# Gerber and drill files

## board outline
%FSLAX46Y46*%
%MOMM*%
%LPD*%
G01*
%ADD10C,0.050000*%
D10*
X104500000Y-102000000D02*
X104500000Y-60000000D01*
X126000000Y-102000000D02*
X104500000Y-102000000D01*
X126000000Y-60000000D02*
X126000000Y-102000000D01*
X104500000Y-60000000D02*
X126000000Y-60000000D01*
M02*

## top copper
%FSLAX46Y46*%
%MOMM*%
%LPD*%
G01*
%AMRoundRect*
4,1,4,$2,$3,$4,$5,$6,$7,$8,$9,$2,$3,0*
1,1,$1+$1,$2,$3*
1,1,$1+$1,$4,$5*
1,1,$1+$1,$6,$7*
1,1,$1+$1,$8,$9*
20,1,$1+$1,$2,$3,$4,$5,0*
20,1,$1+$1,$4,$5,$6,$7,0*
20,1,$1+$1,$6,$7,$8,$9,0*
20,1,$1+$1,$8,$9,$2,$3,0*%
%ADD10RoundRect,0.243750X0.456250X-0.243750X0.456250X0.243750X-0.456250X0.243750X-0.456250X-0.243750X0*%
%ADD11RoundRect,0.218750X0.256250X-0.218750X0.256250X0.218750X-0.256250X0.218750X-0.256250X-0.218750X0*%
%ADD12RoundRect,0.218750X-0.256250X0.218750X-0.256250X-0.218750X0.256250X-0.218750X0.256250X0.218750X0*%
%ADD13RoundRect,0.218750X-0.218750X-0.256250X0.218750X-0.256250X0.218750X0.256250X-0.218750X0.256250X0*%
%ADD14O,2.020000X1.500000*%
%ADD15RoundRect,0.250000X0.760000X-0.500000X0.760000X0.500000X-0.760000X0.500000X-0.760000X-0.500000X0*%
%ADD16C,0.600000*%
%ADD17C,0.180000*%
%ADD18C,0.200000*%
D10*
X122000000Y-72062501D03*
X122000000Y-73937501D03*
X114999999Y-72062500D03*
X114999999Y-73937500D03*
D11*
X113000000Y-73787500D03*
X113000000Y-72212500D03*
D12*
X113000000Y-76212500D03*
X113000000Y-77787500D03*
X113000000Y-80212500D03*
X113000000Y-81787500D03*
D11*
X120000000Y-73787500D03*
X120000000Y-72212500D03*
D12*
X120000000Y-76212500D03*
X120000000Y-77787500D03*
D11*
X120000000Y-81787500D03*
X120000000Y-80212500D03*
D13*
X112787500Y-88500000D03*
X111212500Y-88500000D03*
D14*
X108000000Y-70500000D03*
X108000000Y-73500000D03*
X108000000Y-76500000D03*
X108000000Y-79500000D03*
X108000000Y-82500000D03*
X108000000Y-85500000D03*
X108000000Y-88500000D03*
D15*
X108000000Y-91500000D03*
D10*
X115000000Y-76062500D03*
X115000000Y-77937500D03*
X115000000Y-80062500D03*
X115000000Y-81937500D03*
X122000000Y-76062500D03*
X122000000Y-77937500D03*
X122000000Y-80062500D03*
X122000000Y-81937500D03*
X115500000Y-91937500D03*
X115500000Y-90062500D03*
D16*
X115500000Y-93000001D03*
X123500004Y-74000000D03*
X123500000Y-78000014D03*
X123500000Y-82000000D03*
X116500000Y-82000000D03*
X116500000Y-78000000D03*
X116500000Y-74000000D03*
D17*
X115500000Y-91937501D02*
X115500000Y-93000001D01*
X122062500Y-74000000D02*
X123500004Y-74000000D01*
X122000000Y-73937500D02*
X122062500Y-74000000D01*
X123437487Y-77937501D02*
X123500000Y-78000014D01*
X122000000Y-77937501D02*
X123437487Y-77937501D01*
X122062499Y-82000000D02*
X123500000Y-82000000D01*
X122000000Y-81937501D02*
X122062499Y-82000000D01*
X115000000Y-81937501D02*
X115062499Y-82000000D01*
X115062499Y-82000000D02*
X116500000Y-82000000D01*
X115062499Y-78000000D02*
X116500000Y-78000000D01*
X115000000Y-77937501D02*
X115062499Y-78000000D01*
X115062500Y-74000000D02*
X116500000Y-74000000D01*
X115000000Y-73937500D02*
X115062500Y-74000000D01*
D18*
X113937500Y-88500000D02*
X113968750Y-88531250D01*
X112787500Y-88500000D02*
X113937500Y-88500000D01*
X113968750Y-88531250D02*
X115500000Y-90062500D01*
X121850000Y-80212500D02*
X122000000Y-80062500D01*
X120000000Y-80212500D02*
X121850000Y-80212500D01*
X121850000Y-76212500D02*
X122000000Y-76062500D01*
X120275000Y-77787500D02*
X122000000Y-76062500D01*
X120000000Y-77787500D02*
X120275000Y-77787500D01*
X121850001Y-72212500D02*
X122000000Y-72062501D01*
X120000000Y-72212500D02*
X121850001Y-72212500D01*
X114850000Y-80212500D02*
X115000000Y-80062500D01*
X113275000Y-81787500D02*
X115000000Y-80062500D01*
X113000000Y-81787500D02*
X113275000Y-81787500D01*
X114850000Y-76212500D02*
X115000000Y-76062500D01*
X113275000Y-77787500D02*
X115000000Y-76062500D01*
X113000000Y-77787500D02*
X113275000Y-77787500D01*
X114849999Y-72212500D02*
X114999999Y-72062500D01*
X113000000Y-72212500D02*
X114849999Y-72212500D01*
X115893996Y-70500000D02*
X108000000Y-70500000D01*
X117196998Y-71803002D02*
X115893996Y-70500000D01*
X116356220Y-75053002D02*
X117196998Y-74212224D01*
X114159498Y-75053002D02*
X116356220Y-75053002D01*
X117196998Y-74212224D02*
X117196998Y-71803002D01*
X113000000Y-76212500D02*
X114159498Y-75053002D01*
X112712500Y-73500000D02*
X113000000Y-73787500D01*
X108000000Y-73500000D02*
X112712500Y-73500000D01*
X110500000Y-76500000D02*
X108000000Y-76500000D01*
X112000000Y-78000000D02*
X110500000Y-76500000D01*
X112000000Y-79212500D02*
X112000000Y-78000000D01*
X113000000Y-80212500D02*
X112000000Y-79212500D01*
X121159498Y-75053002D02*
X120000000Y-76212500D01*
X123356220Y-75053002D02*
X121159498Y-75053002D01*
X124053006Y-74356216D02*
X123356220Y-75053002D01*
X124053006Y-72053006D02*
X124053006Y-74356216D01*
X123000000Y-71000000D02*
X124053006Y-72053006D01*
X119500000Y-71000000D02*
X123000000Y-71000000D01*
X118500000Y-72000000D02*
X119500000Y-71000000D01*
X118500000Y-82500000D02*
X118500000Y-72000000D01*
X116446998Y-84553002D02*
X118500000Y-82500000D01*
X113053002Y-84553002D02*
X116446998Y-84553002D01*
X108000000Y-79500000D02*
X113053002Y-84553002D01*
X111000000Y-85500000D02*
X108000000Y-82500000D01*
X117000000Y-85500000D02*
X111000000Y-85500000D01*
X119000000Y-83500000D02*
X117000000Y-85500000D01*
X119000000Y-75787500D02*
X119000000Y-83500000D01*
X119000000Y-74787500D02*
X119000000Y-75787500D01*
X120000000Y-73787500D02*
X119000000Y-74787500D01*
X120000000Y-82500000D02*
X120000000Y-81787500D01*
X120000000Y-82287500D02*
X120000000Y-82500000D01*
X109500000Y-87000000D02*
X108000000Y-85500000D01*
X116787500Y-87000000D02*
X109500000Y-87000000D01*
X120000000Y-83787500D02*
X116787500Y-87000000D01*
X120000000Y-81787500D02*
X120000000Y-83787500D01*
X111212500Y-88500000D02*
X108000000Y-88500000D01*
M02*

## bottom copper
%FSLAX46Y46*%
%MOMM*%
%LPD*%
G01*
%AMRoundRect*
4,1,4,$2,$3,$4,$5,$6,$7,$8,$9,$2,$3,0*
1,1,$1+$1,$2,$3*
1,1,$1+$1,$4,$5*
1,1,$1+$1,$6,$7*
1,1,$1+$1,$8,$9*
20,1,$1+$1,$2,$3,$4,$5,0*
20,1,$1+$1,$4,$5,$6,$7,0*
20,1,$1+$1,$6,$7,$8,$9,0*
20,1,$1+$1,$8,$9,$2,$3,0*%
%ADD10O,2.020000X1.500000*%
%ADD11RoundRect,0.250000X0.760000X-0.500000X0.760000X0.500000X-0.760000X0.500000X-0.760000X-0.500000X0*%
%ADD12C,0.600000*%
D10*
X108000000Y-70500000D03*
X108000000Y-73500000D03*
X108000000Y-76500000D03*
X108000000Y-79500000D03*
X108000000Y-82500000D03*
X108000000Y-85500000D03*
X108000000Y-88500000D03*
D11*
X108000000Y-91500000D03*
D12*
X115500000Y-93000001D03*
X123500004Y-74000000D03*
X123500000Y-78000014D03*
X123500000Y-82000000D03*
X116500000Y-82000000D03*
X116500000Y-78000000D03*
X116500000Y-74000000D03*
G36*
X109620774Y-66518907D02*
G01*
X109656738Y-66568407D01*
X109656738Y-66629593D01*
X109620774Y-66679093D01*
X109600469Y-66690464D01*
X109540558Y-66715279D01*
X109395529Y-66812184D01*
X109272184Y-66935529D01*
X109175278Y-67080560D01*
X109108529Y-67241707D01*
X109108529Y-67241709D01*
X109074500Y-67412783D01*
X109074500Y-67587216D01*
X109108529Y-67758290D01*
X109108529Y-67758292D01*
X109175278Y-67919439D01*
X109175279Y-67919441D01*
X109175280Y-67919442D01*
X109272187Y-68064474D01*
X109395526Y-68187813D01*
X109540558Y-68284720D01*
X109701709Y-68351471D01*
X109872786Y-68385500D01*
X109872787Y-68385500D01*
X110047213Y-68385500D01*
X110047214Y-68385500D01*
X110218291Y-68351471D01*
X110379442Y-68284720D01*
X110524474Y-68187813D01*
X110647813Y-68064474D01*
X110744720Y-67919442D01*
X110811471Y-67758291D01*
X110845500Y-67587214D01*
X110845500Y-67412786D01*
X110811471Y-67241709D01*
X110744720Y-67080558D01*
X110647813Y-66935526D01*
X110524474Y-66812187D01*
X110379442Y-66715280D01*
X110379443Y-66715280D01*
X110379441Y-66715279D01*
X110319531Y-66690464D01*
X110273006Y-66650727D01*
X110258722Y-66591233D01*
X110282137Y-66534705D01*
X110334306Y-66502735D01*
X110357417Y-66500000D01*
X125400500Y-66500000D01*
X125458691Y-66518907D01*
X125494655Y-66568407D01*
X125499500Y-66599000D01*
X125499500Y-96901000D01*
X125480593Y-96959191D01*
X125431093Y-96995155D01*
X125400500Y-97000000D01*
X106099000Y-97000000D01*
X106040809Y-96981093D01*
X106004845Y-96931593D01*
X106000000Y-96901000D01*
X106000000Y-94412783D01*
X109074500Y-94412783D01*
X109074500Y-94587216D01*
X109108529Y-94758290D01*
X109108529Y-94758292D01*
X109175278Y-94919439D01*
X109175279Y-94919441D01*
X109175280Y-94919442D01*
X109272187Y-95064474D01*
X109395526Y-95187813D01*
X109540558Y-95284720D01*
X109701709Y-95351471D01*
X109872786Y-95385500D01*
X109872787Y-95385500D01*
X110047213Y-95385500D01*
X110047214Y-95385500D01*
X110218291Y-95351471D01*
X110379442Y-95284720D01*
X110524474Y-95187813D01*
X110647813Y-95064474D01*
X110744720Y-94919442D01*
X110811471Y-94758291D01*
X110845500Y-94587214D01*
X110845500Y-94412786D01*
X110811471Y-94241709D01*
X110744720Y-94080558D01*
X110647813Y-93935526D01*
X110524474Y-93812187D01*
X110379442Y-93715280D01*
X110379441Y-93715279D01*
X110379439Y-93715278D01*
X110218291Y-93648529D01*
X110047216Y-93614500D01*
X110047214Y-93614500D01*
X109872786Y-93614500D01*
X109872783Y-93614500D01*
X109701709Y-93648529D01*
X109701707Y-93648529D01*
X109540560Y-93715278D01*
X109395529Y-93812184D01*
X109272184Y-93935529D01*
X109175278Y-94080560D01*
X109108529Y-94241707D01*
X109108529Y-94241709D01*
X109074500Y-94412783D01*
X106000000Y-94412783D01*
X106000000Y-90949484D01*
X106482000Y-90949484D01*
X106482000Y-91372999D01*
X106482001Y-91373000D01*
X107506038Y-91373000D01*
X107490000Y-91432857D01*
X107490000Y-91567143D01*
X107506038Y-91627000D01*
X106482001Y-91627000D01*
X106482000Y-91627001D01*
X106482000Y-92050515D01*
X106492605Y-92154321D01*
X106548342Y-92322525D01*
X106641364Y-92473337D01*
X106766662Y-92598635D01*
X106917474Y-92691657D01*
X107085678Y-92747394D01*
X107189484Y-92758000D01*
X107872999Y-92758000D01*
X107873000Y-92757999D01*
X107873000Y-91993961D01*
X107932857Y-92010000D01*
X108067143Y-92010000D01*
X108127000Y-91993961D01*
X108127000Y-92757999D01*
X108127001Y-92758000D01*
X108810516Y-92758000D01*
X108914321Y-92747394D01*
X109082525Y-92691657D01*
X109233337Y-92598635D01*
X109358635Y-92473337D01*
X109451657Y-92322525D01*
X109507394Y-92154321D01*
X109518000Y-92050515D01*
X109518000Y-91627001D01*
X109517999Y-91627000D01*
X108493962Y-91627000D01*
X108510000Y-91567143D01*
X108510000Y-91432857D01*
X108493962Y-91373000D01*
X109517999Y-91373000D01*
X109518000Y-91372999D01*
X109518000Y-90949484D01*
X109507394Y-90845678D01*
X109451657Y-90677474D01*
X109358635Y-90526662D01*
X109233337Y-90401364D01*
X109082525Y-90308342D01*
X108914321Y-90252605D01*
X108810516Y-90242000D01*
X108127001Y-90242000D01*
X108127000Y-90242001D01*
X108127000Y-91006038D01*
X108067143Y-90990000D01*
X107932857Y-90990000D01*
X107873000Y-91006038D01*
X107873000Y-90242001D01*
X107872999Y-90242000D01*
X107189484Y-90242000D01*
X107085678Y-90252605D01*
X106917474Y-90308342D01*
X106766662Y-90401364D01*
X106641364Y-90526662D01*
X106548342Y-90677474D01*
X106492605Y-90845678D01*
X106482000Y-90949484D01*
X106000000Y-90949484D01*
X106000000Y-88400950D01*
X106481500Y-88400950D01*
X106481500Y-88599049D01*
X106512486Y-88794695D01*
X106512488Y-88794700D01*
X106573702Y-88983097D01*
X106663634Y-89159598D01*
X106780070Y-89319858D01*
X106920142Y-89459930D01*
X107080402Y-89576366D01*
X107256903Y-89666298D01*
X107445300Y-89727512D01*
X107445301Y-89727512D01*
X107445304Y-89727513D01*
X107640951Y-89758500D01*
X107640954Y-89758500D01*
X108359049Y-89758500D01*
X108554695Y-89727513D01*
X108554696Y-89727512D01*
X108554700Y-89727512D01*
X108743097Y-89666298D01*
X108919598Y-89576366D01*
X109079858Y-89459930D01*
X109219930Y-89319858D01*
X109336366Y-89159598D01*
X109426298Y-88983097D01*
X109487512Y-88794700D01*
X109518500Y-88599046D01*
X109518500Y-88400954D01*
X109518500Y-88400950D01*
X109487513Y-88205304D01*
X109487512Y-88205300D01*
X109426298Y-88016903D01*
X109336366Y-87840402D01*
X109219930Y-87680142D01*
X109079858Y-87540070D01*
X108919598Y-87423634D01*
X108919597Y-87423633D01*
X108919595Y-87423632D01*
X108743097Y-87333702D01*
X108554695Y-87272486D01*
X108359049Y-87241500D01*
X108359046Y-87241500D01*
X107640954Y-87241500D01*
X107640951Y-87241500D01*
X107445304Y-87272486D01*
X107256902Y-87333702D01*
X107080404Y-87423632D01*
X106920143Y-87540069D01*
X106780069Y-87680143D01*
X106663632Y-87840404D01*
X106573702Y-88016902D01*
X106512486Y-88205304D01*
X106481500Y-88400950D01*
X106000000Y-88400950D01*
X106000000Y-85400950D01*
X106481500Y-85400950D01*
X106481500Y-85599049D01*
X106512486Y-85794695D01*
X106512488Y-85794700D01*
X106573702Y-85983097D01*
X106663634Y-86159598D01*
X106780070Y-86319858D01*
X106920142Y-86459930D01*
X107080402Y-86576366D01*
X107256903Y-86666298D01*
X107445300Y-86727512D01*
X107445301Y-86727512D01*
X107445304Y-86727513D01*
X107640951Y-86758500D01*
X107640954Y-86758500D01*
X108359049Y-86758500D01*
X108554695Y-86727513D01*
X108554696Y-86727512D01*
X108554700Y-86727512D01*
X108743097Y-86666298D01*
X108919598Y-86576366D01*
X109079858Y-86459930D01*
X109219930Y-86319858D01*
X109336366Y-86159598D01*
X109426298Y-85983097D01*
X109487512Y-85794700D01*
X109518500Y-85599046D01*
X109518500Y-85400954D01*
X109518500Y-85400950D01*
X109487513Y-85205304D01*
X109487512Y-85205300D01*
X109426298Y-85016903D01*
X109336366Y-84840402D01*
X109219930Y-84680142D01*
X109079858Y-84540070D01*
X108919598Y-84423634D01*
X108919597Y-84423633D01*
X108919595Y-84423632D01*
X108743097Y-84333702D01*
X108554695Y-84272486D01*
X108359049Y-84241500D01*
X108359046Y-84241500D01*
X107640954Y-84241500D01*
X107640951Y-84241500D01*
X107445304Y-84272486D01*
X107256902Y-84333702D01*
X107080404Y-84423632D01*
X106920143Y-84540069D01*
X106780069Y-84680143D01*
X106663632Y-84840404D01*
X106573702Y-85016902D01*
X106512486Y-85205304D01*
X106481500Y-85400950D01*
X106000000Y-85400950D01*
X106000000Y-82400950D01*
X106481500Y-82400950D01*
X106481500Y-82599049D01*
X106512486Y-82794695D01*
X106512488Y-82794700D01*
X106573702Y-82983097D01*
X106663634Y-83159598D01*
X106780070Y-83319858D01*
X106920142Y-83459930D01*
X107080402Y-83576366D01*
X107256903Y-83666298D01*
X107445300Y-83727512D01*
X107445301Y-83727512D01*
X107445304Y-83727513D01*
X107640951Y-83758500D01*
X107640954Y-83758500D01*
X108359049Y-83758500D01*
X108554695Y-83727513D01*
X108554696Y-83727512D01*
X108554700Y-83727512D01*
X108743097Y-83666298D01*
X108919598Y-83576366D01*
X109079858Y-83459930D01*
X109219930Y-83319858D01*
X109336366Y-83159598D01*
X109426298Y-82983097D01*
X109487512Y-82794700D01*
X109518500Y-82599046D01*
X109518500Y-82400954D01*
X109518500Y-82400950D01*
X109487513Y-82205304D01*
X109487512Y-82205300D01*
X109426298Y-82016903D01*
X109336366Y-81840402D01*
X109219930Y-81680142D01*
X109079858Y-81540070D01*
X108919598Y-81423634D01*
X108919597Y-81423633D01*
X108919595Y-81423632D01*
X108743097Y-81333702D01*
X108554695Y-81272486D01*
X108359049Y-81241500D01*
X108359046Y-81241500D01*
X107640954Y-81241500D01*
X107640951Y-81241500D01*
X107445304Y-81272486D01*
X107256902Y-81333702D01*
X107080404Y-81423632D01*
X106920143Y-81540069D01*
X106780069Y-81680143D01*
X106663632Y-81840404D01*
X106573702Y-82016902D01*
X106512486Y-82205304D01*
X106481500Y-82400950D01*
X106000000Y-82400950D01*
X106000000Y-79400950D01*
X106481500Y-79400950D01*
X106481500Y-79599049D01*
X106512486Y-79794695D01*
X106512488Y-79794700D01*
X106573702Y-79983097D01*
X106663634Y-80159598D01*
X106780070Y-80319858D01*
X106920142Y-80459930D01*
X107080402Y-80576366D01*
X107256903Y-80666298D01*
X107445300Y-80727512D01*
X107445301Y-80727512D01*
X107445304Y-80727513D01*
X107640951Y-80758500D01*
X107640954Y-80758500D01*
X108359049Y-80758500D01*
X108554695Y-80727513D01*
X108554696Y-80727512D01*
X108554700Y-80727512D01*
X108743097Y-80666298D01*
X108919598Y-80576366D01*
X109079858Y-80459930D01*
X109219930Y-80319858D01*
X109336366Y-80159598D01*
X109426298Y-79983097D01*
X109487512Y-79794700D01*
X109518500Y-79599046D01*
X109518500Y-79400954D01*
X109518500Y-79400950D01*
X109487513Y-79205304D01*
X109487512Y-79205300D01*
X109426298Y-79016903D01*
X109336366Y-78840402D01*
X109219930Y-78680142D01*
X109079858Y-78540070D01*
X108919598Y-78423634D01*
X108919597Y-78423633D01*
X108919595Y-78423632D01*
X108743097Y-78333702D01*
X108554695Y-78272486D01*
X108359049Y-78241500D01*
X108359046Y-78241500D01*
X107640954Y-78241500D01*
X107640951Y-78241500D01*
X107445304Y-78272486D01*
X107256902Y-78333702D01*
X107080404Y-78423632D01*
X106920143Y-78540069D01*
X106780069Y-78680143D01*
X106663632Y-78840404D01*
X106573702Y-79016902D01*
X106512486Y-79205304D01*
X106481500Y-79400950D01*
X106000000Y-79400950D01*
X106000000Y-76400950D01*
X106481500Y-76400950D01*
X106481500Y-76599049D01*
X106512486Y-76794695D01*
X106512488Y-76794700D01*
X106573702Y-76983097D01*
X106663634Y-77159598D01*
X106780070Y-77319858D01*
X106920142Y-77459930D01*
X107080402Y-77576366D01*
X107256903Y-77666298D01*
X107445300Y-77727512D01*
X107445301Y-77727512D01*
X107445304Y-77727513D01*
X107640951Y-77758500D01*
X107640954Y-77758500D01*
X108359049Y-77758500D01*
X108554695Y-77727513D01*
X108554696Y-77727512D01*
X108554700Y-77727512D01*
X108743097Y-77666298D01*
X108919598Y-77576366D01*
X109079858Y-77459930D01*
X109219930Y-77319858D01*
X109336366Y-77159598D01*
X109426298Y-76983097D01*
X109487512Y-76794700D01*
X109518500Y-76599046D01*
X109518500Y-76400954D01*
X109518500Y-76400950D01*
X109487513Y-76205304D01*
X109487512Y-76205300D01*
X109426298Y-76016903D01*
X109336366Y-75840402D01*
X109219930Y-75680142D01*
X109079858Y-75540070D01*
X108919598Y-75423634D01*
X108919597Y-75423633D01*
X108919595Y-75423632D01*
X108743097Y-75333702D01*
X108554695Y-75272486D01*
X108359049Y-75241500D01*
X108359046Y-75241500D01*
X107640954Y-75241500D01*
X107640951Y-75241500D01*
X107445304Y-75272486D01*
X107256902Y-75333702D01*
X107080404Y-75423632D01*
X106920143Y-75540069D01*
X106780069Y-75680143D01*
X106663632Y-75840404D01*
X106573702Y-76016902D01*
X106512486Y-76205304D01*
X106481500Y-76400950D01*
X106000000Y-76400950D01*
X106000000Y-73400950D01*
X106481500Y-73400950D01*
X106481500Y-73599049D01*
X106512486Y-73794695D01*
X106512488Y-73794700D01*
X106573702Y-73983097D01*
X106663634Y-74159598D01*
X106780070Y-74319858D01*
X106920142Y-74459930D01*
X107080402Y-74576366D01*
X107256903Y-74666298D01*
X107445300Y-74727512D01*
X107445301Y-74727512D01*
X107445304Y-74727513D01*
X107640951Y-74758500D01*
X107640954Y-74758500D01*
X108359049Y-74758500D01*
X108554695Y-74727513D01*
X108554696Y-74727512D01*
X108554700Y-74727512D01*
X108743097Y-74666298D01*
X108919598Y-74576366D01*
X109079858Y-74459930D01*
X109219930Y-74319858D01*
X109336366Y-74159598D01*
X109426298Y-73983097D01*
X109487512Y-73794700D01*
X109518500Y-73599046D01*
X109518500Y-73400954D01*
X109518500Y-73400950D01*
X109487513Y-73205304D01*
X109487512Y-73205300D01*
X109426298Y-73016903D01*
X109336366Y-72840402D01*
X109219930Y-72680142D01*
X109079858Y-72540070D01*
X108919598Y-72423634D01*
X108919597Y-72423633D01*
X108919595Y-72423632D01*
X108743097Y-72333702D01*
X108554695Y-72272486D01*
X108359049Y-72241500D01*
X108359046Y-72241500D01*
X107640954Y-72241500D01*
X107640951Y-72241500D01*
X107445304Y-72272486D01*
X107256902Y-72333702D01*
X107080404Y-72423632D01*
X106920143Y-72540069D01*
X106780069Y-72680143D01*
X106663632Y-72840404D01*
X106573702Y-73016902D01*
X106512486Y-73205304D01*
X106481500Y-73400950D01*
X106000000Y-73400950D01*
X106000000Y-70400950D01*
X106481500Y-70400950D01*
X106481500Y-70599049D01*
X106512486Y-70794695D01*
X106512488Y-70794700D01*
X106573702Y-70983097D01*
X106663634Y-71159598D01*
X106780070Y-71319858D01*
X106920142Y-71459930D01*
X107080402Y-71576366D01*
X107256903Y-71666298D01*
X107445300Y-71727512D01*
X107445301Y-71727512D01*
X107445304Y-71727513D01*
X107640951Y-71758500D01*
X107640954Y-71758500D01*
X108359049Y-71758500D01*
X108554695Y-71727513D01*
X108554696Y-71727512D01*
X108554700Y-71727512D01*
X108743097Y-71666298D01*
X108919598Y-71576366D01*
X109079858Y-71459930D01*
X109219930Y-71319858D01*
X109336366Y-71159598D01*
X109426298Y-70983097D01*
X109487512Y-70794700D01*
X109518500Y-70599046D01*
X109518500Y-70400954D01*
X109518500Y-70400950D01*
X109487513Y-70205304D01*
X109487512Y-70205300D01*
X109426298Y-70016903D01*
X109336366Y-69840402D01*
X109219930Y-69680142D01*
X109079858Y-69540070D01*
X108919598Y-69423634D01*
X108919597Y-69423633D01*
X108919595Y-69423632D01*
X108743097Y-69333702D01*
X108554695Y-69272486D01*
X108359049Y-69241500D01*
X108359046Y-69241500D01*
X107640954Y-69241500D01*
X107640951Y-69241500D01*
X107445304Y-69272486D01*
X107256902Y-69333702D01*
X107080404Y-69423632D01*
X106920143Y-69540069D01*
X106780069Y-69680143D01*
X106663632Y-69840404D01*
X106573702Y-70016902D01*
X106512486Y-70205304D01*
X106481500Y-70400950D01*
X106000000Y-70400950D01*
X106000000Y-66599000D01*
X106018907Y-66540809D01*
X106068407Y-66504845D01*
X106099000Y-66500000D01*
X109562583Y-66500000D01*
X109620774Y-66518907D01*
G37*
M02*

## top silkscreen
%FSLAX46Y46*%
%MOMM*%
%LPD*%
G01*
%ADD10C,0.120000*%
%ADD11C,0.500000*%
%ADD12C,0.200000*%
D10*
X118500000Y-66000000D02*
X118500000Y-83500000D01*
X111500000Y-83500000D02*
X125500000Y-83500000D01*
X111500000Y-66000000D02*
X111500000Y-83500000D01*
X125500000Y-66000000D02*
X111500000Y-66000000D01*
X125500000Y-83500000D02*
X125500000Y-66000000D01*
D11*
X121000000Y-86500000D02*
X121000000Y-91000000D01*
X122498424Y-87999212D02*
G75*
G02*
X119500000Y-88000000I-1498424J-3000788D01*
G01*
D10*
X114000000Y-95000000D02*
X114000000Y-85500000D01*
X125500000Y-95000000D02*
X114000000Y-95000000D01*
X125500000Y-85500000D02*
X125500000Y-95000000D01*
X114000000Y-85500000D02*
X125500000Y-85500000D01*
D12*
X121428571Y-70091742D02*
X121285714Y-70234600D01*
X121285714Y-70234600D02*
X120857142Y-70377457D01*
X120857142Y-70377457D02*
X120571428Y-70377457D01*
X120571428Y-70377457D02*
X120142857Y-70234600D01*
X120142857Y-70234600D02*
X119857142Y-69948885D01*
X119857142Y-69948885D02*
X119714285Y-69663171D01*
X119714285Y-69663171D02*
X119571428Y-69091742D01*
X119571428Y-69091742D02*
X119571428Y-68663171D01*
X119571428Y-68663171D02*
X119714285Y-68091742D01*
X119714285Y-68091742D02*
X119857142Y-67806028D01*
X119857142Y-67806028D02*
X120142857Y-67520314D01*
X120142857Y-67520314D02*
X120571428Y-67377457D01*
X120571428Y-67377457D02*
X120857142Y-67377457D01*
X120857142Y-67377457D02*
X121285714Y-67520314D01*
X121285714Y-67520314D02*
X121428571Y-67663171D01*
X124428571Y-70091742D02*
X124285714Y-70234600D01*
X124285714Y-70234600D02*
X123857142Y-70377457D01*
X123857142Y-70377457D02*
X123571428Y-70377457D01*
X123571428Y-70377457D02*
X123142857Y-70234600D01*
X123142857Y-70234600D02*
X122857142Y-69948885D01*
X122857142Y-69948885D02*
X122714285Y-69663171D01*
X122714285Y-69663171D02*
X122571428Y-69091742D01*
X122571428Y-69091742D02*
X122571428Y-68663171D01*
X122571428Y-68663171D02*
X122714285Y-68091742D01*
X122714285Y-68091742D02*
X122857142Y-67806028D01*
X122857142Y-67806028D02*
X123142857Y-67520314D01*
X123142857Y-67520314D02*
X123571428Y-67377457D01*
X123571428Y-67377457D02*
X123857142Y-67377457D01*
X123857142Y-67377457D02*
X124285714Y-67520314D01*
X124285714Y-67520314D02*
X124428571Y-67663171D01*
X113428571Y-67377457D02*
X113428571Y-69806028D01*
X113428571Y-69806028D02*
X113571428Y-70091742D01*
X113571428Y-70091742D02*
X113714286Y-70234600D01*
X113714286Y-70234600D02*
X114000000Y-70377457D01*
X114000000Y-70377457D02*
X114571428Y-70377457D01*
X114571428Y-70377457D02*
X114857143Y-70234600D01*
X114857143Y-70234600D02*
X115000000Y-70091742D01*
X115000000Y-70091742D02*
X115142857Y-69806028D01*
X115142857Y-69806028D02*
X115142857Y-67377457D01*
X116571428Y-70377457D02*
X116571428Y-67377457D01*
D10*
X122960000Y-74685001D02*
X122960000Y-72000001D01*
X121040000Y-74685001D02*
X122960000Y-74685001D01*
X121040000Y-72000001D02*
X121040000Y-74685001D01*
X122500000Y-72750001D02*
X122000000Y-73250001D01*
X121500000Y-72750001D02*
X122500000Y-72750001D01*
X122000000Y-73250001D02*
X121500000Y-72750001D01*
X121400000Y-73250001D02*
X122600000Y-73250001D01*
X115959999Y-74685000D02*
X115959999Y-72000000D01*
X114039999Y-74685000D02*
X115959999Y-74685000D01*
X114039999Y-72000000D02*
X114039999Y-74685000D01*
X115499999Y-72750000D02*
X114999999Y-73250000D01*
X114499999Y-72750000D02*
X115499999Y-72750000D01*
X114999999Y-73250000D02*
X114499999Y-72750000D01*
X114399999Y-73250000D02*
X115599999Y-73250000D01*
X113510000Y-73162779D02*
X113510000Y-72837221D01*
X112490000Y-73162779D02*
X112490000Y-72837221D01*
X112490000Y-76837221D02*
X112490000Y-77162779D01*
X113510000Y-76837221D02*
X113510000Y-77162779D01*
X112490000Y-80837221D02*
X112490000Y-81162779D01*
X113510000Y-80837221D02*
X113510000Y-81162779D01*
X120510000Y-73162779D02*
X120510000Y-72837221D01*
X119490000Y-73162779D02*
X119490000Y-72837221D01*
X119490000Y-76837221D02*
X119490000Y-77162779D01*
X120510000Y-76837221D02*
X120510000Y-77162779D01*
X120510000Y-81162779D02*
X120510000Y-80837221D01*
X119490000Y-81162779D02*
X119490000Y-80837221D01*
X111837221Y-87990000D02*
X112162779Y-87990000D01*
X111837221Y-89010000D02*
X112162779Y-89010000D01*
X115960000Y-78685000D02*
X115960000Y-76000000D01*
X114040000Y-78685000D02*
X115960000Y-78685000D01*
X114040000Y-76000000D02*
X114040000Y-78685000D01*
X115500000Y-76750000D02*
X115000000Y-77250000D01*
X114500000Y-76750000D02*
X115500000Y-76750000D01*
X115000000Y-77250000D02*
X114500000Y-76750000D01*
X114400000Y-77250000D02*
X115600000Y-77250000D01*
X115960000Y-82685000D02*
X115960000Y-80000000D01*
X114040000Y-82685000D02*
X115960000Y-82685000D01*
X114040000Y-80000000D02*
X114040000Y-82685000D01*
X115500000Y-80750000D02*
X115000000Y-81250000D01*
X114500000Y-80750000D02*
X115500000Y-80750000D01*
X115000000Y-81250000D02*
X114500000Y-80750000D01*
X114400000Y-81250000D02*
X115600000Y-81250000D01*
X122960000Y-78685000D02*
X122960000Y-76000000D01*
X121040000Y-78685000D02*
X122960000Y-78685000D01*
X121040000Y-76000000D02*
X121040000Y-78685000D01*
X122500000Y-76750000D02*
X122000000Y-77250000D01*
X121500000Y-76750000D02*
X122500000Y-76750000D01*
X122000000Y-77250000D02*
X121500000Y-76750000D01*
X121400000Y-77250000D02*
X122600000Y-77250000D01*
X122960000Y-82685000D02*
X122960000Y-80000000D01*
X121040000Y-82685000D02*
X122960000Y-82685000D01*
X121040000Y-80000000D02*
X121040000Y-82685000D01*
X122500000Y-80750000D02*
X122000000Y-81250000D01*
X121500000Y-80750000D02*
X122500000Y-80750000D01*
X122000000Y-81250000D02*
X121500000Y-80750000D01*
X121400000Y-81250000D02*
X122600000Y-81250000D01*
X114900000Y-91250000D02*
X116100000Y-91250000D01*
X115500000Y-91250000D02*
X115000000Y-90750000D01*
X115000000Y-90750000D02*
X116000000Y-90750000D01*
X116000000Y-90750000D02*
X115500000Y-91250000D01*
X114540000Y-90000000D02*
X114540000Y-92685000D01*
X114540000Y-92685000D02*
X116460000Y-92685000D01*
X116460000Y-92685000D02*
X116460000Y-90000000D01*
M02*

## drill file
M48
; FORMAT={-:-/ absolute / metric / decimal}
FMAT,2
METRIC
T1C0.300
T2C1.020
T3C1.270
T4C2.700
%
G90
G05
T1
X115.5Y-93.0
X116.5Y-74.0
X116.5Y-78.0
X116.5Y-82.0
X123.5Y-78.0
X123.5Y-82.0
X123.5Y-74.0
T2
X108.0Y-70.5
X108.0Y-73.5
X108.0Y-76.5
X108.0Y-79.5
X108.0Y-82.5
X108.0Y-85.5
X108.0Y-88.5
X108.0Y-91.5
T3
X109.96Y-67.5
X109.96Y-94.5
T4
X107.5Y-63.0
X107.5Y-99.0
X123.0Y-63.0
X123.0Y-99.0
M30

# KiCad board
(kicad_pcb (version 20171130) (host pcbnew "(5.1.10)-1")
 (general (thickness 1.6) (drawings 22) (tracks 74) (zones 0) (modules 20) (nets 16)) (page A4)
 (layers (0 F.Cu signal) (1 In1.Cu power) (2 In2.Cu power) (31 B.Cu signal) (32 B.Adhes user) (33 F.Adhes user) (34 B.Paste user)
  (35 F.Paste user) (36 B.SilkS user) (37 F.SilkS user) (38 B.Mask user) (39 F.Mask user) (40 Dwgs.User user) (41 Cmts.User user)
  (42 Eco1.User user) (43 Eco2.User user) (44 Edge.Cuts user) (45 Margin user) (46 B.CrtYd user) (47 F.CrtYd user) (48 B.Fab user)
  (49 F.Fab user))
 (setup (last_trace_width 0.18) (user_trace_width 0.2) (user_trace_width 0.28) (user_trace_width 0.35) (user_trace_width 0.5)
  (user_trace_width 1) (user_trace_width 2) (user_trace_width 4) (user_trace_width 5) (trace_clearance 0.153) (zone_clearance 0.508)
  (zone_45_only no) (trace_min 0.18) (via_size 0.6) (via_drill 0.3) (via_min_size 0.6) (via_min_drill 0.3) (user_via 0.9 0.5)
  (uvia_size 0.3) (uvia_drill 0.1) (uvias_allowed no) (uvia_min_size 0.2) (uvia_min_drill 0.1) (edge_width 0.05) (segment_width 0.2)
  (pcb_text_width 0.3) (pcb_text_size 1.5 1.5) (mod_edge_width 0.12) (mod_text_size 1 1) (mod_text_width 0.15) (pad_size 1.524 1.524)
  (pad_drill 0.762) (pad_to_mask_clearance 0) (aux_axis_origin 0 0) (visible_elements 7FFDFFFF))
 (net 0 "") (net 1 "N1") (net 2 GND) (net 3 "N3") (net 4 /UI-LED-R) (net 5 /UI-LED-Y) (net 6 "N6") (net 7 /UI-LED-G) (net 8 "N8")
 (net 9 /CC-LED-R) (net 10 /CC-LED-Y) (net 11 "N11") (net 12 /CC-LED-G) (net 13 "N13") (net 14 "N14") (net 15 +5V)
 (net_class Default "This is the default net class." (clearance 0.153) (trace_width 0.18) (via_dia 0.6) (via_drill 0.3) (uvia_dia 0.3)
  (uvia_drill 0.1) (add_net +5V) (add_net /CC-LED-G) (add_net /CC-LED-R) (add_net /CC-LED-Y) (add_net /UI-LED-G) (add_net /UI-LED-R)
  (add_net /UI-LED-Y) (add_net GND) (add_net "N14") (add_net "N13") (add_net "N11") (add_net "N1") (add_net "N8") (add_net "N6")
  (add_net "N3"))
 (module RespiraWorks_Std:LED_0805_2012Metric (layer F.Cu) (at 122 73.000001 90)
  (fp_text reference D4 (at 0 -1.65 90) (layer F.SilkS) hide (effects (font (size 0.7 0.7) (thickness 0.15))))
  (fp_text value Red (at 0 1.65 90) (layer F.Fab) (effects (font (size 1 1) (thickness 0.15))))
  (fp_line (start -1.685 0.96) (end 1 0.96) (layer F.SilkS) (width 0.12))
  (fp_line (start -1.685 -0.96) (end -1.685 0.96) (layer F.SilkS) (width 0.12))
  (fp_line (start 1 -0.96) (end -1.685 -0.96) (layer F.SilkS) (width 0.12))
  (fp_line (start 0.25 0.5) (end -0.25 0) (layer F.SilkS) (width 0.12))
  (fp_line (start 0.25 -0.5) (end 0.25 0.5) (layer F.SilkS) (width 0.12))
  (fp_line (start -0.25 0) (end 0.25 -0.5) (layer F.SilkS) (width 0.12))
  (fp_line (start -0.25 -0.6) (end -0.25 0.6) (layer F.SilkS) (width 0.12))
  (pad 2 smd roundrect (at 0.9375 0 90) (size 0.975 1.4) (layers F.Cu F.Paste F.Mask) (roundrect_rratio 0.25) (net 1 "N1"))
  (pad 1 smd roundrect (at -0.9375 0 90) (size 0.975 1.4) (layers F.Cu F.Paste F.Mask) (roundrect_rratio 0.25) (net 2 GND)))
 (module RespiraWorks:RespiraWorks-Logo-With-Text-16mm (layer B.Cu) (at 117.5 78 180)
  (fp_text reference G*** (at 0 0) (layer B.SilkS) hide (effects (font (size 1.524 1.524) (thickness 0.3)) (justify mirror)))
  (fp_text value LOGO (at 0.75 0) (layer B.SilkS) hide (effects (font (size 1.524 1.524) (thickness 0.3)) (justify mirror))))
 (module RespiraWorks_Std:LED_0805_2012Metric (layer F.Cu) (at 114.999999 73 90)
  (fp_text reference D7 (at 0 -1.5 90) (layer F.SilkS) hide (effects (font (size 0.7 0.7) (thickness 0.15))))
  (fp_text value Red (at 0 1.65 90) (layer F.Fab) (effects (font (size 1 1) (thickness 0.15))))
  (fp_line (start -1.685 0.96) (end 1 0.96) (layer F.SilkS) (width 0.12))
  (fp_line (start -1.685 -0.96) (end -1.685 0.96) (layer F.SilkS) (width 0.12))
  (fp_line (start 1 -0.96) (end -1.685 -0.96) (layer F.SilkS) (width 0.12))
  (fp_line (start 0.25 0.5) (end -0.25 0) (layer F.SilkS) (width 0.12))
  (fp_line (start 0.25 -0.5) (end 0.25 0.5) (layer F.SilkS) (width 0.12))
  (fp_line (start -0.25 0) (end 0.25 -0.5) (layer F.SilkS) (width 0.12))
  (fp_line (start -0.25 -0.6) (end -0.25 0.6) (layer F.SilkS) (width 0.12))
  (pad 2 smd roundrect (at 0.9375 0 90) (size 0.975 1.4) (layers F.Cu F.Paste F.Mask) (roundrect_rratio 0.25) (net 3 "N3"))
  (pad 1 smd roundrect (at -0.9375 0 90) (size 0.975 1.4) (layers F.Cu F.Paste F.Mask) (roundrect_rratio 0.25) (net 2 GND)))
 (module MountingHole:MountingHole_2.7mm (layer F.Cu) (at 123 99)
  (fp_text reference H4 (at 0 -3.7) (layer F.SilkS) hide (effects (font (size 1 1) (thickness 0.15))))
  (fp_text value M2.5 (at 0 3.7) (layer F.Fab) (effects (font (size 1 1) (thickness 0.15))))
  (pad 1 np_thru_hole circle (at 0 0) (size 2.7 2.7) (drill 2.7) (layers *.Cu *.Mask)))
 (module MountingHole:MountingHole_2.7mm (layer F.Cu) (at 123 63)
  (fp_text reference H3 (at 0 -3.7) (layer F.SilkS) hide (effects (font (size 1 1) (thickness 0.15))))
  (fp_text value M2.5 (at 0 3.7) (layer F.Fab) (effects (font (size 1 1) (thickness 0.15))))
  (pad 1 np_thru_hole circle (at 0 0) (size 2.7 2.7) (drill 2.7) (layers *.Cu *.Mask)))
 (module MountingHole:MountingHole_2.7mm (layer F.Cu) (at 107.5 99)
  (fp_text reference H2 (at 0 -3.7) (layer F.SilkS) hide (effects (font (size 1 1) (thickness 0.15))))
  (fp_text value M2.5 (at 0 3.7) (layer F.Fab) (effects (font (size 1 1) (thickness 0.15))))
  (pad 1 np_thru_hole circle (at 0 0) (size 2.7 2.7) (drill 2.7) (layers *.Cu *.Mask)))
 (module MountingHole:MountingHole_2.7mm (layer F.Cu) (at 107.5 63)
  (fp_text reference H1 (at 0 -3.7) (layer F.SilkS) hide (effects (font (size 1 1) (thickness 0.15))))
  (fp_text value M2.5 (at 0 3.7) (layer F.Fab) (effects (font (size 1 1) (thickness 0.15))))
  (pad 1 np_thru_hole circle (at 0 0) (size 2.7 2.7) (drill 2.7) (layers *.Cu *.Mask)))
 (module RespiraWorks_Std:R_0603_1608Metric (layer F.Cu) (at 113 73 90)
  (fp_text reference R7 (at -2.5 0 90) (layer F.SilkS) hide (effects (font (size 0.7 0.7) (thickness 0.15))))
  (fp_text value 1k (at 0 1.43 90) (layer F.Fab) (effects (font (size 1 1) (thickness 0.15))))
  (fp_line (start -0.162779 0.51) (end 0.162779 0.51) (layer F.SilkS) (width 0.12))
  (fp_line (start -0.162779 -0.51) (end 0.162779 -0.51) (layer F.SilkS) (width 0.12))
  (pad 1 smd roundrect (at -0.7875 0 90) (size 0.875 0.95) (layers F.Cu F.Paste F.Mask) (roundrect_rratio 0.25) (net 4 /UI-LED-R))
  (pad 2 smd roundrect (at 0.7875 0 90) (size 0.875 0.95) (layers F.Cu F.Paste F.Mask) (roundrect_rratio 0.25) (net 3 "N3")))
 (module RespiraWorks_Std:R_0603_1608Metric (layer F.Cu) (at 113 77 270)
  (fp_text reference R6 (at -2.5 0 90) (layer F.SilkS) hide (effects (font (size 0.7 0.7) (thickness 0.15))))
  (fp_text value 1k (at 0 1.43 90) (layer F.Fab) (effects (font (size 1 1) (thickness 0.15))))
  (fp_line (start -0.162779 0.51) (end 0.162779 0.51) (layer F.SilkS) (width 0.12))
  (fp_line (start -0.162779 -0.51) (end 0.162779 -0.51) (layer F.SilkS) (width 0.12))
  (pad 1 smd roundrect (at -0.7875 0 270) (size 0.875 0.95) (layers F.Cu F.Paste F.Mask) (roundrect_rratio 0.25) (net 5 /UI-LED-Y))
  (pad 2 smd roundrect (at 0.7875 0 270) (size 0.875 0.95) (layers F.Cu F.Paste F.Mask) (roundrect_rratio 0.25) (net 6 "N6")))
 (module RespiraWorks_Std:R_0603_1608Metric (layer F.Cu) (at 113 81 270)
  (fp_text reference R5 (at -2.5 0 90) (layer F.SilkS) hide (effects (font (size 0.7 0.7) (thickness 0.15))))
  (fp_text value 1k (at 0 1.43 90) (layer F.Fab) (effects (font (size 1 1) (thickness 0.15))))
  (fp_line (start -0.162779 0.51) (end 0.162779 0.51) (layer F.SilkS) (width 0.12))
  (fp_line (start -0.162779 -0.51) (end 0.162779 -0.51) (layer F.SilkS) (width 0.12))
  (pad 1 smd roundrect (at -0.7875 0 270) (size 0.875 0.95) (layers F.Cu F.Paste F.Mask) (roundrect_rratio 0.25) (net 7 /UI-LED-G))
  (pad 2 smd roundrect (at 0.7875 0 270) (size 0.875 0.95) (layers F.Cu F.Paste F.Mask) (roundrect_rratio 0.25) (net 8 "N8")))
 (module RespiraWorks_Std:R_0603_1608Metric (layer F.Cu) (at 120 73 90)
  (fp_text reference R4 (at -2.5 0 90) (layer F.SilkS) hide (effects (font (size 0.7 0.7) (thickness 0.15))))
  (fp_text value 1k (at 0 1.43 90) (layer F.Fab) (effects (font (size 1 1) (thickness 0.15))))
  (fp_line (start -0.162779 0.51) (end 0.162779 0.51) (layer F.SilkS) (width 0.12))
  (fp_line (start -0.162779 -0.51) (end 0.162779 -0.51) (layer F.SilkS) (width 0.12))
  (pad 1 smd roundrect (at -0.7875 0 90) (size 0.875 0.95) (layers F.Cu F.Paste F.Mask) (roundrect_rratio 0.25) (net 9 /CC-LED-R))
  (pad 2 smd roundrect (at 0.7875 0 90) (size 0.875 0.95) (layers F.Cu F.Paste F.Mask) (roundrect_rratio 0.25) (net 1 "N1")))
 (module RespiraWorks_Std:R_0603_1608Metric (layer F.Cu) (at 120 77 270)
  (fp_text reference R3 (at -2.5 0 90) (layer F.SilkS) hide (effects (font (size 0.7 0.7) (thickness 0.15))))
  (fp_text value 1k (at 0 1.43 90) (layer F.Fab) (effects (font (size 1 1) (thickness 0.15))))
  (fp_line (start -0.162779 0.51) (end 0.162779 0.51) (layer F.SilkS) (width 0.12))
  (fp_line (start -0.162779 -0.51) (end 0.162779 -0.51) (layer F.SilkS) (width 0.12))
  (pad 1 smd roundrect (at -0.7875 0 270) (size 0.875 0.95) (layers F.Cu F.Paste F.Mask) (roundrect_rratio 0.25) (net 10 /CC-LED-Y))
  (pad 2 smd roundrect (at 0.7875 0 270) (size 0.875 0.95) (layers F.Cu F.Paste F.Mask) (roundrect_rratio 0.25) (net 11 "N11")))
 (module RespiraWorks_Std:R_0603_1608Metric (layer F.Cu) (at 120 81 90)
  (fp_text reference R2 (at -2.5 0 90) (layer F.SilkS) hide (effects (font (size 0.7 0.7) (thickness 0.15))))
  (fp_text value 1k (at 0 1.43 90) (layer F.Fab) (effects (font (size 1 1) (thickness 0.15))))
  (fp_line (start -0.162779 0.51) (end 0.162779 0.51) (layer F.SilkS) (width 0.12))
  (fp_line (start -0.162779 -0.51) (end 0.162779 -0.51) (layer F.SilkS) (width 0.12))
  (pad 1 smd roundrect (at -0.7875 0 90) (size 0.875 0.95) (layers F.Cu F.Paste F.Mask) (roundrect_rratio 0.25) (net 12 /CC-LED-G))
  (pad 2 smd roundrect (at 0.7875 0 90) (size 0.875 0.95) (layers F.Cu F.Paste F.Mask) (roundrect_rratio 0.25) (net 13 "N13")))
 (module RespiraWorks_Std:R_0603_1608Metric (layer F.Cu) (at 112 88.5)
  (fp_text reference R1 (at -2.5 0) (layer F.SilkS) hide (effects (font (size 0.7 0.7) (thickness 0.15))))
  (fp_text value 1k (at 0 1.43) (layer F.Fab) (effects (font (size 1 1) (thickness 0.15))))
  (fp_line (start -0.162779 -0.51) (end 0.162779 -0.51) (layer F.SilkS) (width 0.12))
  (fp_line (start -0.162779 0.51) (end 0.162779 0.51) (layer F.SilkS) (width 0.12))
  (pad 2 smd roundrect (at 0.7875 0) (size 0.875 0.95) (layers F.Cu F.Paste F.Mask) (roundrect_rratio 0.25) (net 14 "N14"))
  (pad 1 smd roundrect (at -0.7875 0) (size 0.875 0.95) (layers F.Cu F.Paste F.Mask) (roundrect_rratio 0.25) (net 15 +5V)))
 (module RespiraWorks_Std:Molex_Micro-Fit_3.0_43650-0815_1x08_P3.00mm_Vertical (layer B.Cu) (at 108 91.5 90)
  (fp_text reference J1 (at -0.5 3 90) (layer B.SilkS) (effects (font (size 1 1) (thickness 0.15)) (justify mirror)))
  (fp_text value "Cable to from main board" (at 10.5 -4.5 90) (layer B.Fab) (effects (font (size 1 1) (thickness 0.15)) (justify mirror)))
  (pad 8 thru_hole oval (at 21 0 90) (size 1.5 2.02) (drill 1.02) (layers *.Cu *.Mask) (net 5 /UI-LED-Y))
  (pad 7 thru_hole oval (at 18 0 90) (size 1.5 2.02) (drill 1.02) (layers *.Cu *.Mask) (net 4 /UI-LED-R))
  (pad 6 thru_hole oval (at 15 0 90) (size 1.5 2.02) (drill 1.02) (layers *.Cu *.Mask) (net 7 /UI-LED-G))
  (pad 5 thru_hole oval (at 12 0 90) (size 1.5 2.02) (drill 1.02) (layers *.Cu *.Mask) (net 10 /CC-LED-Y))
  (pad 4 thru_hole oval (at 9 0 90) (size 1.5 2.02) (drill 1.02) (layers *.Cu *.Mask) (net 9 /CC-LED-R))
  (pad 3 thru_hole oval (at 6 0 90) (size 1.5 2.02) (drill 1.02) (layers *.Cu *.Mask) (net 12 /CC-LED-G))
  (pad 2 thru_hole oval (at 3 0 90) (size 1.5 2.02) (drill 1.02) (layers *.Cu *.Mask) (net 15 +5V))
  (pad 1 thru_hole roundrect (at 0 0 90) (size 1.5 2.02) (drill 1.02) (layers *.Cu *.Mask) (roundrect_rratio 0.1666666666666667) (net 2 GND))
  (pad "" np_thru_hole circle (at 24 1.96 90) (size 1.27 1.27) (drill 1.27) (layers *.Cu *.Mask))
  (pad "" np_thru_hole circle (at -3 1.96 90) (size 1.27 1.27) (drill 1.27) (layers *.Cu *.Mask)))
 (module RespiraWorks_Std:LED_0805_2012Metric (layer F.Cu) (at 115 77 90)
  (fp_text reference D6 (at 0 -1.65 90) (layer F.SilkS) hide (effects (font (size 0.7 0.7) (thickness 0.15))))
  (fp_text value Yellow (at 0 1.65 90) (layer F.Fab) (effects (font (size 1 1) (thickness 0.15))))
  (fp_line (start -1.685 0.96) (end 1 0.96) (layer F.SilkS) (width 0.12))
  (fp_line (start -1.685 -0.96) (end -1.685 0.96) (layer F.SilkS) (width 0.12))
  (fp_line (start 1 -0.96) (end -1.685 -0.96) (layer F.SilkS) (width 0.12))
  (fp_line (start 0.25 0.5) (end -0.25 0) (layer F.SilkS) (width 0.12))
  (fp_line (start 0.25 -0.5) (end 0.25 0.5) (layer F.SilkS) (width 0.12))
  (fp_line (start -0.25 0) (end 0.25 -0.5) (layer F.SilkS) (width 0.12))
  (fp_line (start -0.25 -0.6) (end -0.25 0.6) (layer F.SilkS) (width 0.12))
  (pad 2 smd roundrect (at 0.9375 0 90) (size 0.975 1.4) (layers F.Cu F.Paste F.Mask) (roundrect_rratio 0.25) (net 6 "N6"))
  (pad 1 smd roundrect (at -0.9375 0 90) (size 0.975 1.4) (layers F.Cu F.Paste F.Mask) (roundrect_rratio 0.25) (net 2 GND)))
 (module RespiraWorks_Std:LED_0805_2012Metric (layer F.Cu) (at 115 81 90)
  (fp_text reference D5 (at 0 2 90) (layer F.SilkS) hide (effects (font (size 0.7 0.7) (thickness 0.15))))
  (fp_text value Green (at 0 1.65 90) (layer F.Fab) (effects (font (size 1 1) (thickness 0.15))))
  (fp_line (start -1.685 0.96) (end 1 0.96) (layer F.SilkS) (width 0.12))
  (fp_line (start -1.685 -0.96) (end -1.685 0.96) (layer F.SilkS) (width 0.12))
  (fp_line (start 1 -0.96) (end -1.685 -0.96) (layer F.SilkS) (width 0.12))
  (fp_line (start 0.25 0.5) (end -0.25 0) (layer F.SilkS) (width 0.12))
  (fp_line (start 0.25 -0.5) (end 0.25 0.5) (layer F.SilkS) (width 0.12))
  (fp_line (start -0.25 0) (end 0.25 -0.5) (layer F.SilkS) (width 0.12))
  (fp_line (start -0.25 -0.6) (end -0.25 0.6) (layer F.SilkS) (width 0.12))
  (pad 2 smd roundrect (at 0.9375 0 90) (size 0.975 1.4) (layers F.Cu F.Paste F.Mask) (roundrect_rratio 0.25) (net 8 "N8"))
  (pad 1 smd roundrect (at -0.9375 0 90) (size 0.975 1.4) (layers F.Cu F.Paste F.Mask) (roundrect_rratio 0.25) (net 2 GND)))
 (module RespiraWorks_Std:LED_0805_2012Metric (layer F.Cu) (at 122 77 90)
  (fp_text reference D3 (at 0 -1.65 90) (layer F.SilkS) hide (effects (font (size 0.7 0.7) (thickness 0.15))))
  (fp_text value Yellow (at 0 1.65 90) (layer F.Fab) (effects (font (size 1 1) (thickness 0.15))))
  (fp_line (start -1.685 0.96) (end 1 0.96) (layer F.SilkS) (width 0.12))
  (fp_line (start -1.685 -0.96) (end -1.685 0.96) (layer F.SilkS) (width 0.12))
  (fp_line (start 1 -0.96) (end -1.685 -0.96) (layer F.SilkS) (width 0.12))
  (fp_line (start 0.25 0.5) (end -0.25 0) (layer F.SilkS) (width 0.12))
  (fp_line (start 0.25 -0.5) (end 0.25 0.5) (layer F.SilkS) (width 0.12))
  (fp_line (start -0.25 0) (end 0.25 -0.5) (layer F.SilkS) (width 0.12))
  (fp_line (start -0.25 -0.6) (end -0.25 0.6) (layer F.SilkS) (width 0.12))
  (pad 2 smd roundrect (at 0.9375 0 90) (size 0.975 1.4) (layers F.Cu F.Paste F.Mask) (roundrect_rratio 0.25) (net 11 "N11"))
  (pad 1 smd roundrect (at -0.9375 0 90) (size 0.975 1.4) (layers F.Cu F.Paste F.Mask) (roundrect_rratio 0.25) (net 2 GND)))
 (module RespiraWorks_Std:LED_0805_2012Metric (layer F.Cu) (at 122 81 90)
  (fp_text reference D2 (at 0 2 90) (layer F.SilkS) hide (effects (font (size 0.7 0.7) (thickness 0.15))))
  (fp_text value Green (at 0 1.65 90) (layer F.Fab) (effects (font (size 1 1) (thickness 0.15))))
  (fp_line (start -1.685 0.96) (end 1 0.96) (layer F.SilkS) (width 0.12))
  (fp_line (start -1.685 -0.96) (end -1.685 0.96) (layer F.SilkS) (width 0.12))
  (fp_line (start 1 -0.96) (end -1.685 -0.96) (layer F.SilkS) (width 0.12))
  (fp_line (start 0.25 0.5) (end -0.25 0) (layer F.SilkS) (width 0.12))
  (fp_line (start 0.25 -0.5) (end 0.25 0.5) (layer F.SilkS) (width 0.12))
  (fp_line (start -0.25 0) (end 0.25 -0.5) (layer F.SilkS) (width 0.12))
  (fp_line (start -0.25 -0.6) (end -0.25 0.6) (layer F.SilkS) (width 0.12))
  (pad 2 smd roundrect (at 0.9375 0 90) (size 0.975 1.4) (layers F.Cu F.Paste F.Mask) (roundrect_rratio 0.25) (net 13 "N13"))
  (pad 1 smd roundrect (at -0.9375 0 90) (size 0.975 1.4) (layers F.Cu F.Paste F.Mask) (roundrect_rratio 0.25) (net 2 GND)))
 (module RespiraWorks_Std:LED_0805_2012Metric (layer F.Cu) (at 115.5 91 90)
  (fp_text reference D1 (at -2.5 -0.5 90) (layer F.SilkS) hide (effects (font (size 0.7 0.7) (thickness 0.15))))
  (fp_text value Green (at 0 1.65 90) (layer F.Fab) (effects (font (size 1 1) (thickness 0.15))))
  (fp_line (start -0.25 -0.6) (end -0.25 0.6) (layer F.SilkS) (width 0.12))
  (fp_line (start -0.25 0) (end 0.25 -0.5) (layer F.SilkS) (width 0.12))
  (fp_line (start 0.25 -0.5) (end 0.25 0.5) (layer F.SilkS) (width 0.12))
  (fp_line (start 0.25 0.5) (end -0.25 0) (layer F.SilkS) (width 0.12))
  (fp_line (start 1 -0.96) (end -1.685 -0.96) (layer F.SilkS) (width 0.12))
  (fp_line (start -1.685 -0.96) (end -1.685 0.96) (layer F.SilkS) (width 0.12))
  (fp_line (start -1.685 0.96) (end 1 0.96) (layer F.SilkS) (width 0.12))
  (pad 1 smd roundrect (at -0.9375 0 90) (size 0.975 1.4) (layers F.Cu F.Paste F.Mask) (roundrect_rratio 0.25) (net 2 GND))
  (pad 2 smd roundrect (at 0.9375 0 90) (size 0.975 1.4) (layers F.Cu F.Paste F.Mask) (roundrect_rratio 0.25) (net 14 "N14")))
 (gr_line (start 118.5 66) (end 118.5 83.5) (layer F.SilkS) (width 0.12))
 (gr_line (start 111.5 83.5) (end 125.5 83.5) (layer F.SilkS) (width 0.12))
 (gr_line (start 111.5 66) (end 111.5 83.5) (layer F.SilkS) (width 0.12))
 (gr_line (start 125.5 66) (end 111.5 66) (layer F.SilkS) (width 0.12))
 (gr_line (start 125.5 83.5) (end 125.5 66) (layer F.SilkS) (width 0.12))
 (gr_line (start 121 86.5) (end 121 91) (layer F.SilkS) (width 0.5))
 (gr_arc (start 121 91) (end 119.5 88) (angle -306.9) (layer F.SilkS) (width 0.5))
 (gr_line (start 104.5 102) (end 104.5 60) (layer Edge.Cuts) (width 0.05))
 (gr_line (start 126 102) (end 104.5 102) (layer Edge.Cuts) (width 0.05))
 (gr_line (start 126 60) (end 126 102) (layer Edge.Cuts) (width 0.05))
 (gr_line (start 104.5 60) (end 126 60) (layer Edge.Cuts) (width 0.05))
 (gr_line (start 114 95) (end 114 85.5) (layer F.SilkS) (width 0.12))
 (gr_line (start 125.5 95) (end 114 95) (layer F.SilkS) (width 0.12))
 (gr_line (start 125.5 85.5) (end 125.5 95) (layer F.SilkS) (width 0.12))
 (gr_line (start 114 85.5) (end 125.5 85.5) (layer F.SilkS) (width 0.12))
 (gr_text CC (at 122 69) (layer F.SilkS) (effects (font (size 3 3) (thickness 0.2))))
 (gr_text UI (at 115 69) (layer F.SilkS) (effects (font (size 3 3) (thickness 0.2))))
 (segment (start 115.5 91.937501) (end 115.5 93.000001) (width 0.18) (layer F.Cu) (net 2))
 (via (at 115.5 93.000001) (size 0.6) (drill 0.3) (layers F.Cu B.Cu) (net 2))
 (via (at 123.500004 74) (size 0.6) (drill 0.3) (layers F.Cu B.Cu) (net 2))
 (segment (start 122.0625 74) (end 123.500004 74) (width 0.18) (layer F.Cu) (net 2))
 (segment (start 122 73.9375) (end 122.0625 74) (width 0.18) (layer F.Cu) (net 2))
 (via (at 123.5 78.000014) (size 0.6) (drill 0.3) (layers F.Cu B.Cu) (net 2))
 (segment (start 123.437487 77.937501) (end 123.5 78.000014) (width 0.18) (layer F.Cu) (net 2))
 (segment (start 122 77.937501) (end 123.437487 77.937501) (width 0.18) (layer F.Cu) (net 2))
 (via (at 123.5 82) (size 0.6) (drill 0.3) (layers F.Cu B.Cu) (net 2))
 (segment (start 122.062499 82) (end 123.5 82) (width 0.18) (layer F.Cu) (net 2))
 (segment (start 122 81.937501) (end 122.062499 82) (width 0.18) (layer F.Cu) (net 2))
 (via (at 116.5 82) (size 0.6) (drill 0.3) (layers F.Cu B.Cu) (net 2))
 (segment (start 115 81.937501) (end 115.062499 82) (width 0.18) (layer F.Cu) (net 2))
 (segment (start 115.062499 82) (end 116.5 82) (width 0.18) (layer F.Cu) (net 2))
 (segment (start 115.062499 78) (end 116.5 78) (width 0.18) (layer F.Cu) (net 2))
 (segment (start 115 77.937501) (end 115.062499 78) (width 0.18) (layer F.Cu) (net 2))
 (via (at 116.5 78) (size 0.6) (drill 0.3) (layers F.Cu B.Cu) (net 2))
 (segment (start 115.0625 74) (end 116.5 74) (width 0.18) (layer F.Cu) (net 2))
 (via (at 116.5 74) (size 0.6) (drill 0.3) (layers F.Cu B.Cu) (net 2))
 (segment (start 115 73.9375) (end 115.0625 74) (width 0.18) (layer F.Cu) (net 2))
 (segment (start 113.9375 88.5) (end 113.96875 88.53125) (width 0.2) (layer F.Cu) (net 14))
 (segment (start 112.7875 88.5) (end 113.9375 88.5) (width 0.2) (layer F.Cu) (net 14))
 (segment (start 113.96875 88.53125) (end 115.5 90.0625) (width 0.2) (layer F.Cu) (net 14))
 (segment (start 121.85 80.2125) (end 122 80.0625) (width 0.2) (layer F.Cu) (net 13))
 (segment (start 120 80.2125) (end 121.85 80.2125) (width 0.2) (layer F.Cu) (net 13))
 (segment (start 121.85 76.2125) (end 122 76.0625) (width 0.2) (layer F.Cu) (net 11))
 (segment (start 120.275 77.7875) (end 122 76.0625) (width 0.2) (layer F.Cu) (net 11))
 (segment (start 120 77.7875) (end 120.275 77.7875) (width 0.2) (layer F.Cu) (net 11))
 (segment (start 121.850001 72.2125) (end 122 72.062501) (width 0.2) (layer F.Cu) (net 1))
 (segment (start 120 72.2125) (end 121.850001 72.2125) (width 0.2) (layer F.Cu) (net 1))
 (segment (start 114.85 80.2125) (end 115 80.0625) (width 0.2) (layer F.Cu) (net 8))
 (segment (start 113.275 81.7875) (end 115 80.0625) (width 0.2) (layer F.Cu) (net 8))
 (segment (start 113 81.7875) (end 113.275 81.7875) (width 0.2) (layer F.Cu) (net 8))
 (segment (start 114.85 76.2125) (end 115 76.0625) (width 0.2) (layer F.Cu) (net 6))
 (segment (start 113.275 77.7875) (end 115 76.0625) (width 0.2) (layer F.Cu) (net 6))
 (segment (start 113 77.7875) (end 113.275 77.7875) (width 0.2) (layer F.Cu) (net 6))
 (segment (start 114.849999 72.2125) (end 114.999999 72.0625) (width 0.2) (layer F.Cu) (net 3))
 (segment (start 113 72.2125) (end 114.849999 72.2125) (width 0.2) (layer F.Cu) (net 3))
 (segment (start 115.893996 70.5) (end 108 70.5) (width 0.2) (layer F.Cu) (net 5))
 (segment (start 117.196998 71.803002) (end 115.893996 70.5) (width 0.2) (layer F.Cu) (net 5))
 (segment (start 116.35622 75.053002) (end 117.196998 74.212224) (width 0.2) (layer F.Cu) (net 5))
 (segment (start 114.159498 75.053002) (end 116.35622 75.053002) (width 0.2) (layer F.Cu) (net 5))
 (segment (start 117.196998 74.212224) (end 117.196998 71.803002) (width 0.2) (layer F.Cu) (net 5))
 (segment (start 113 76.2125) (end 114.159498 75.053002) (width 0.2) (layer F.Cu) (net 5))
 (segment (start 112.7125 73.5) (end 113 73.7875) (width 0.2) (layer F.Cu) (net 4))
 (segment (start 108 73.5) (end 112.7125 73.5) (width 0.2) (layer F.Cu) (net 4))
 (segment (start 110.5 76.5) (end 108 76.5) (width 0.2) (layer F.Cu) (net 7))
 (segment (start 112 78) (end 110.5 76.5) (width 0.2) (layer F.Cu) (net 7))
 (segment (start 112 79.2125) (end 112 78) (width 0.2) (layer F.Cu) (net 7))
 (segment (start 113 80.2125) (end 112 79.2125) (width 0.2) (layer F.Cu) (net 7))
 (segment (start 121.159498 75.053002) (end 120 76.2125) (width 0.2) (layer F.Cu) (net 10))
 (segment (start 123.35622 75.053002) (end 121.159498 75.053002) (width 0.2) (layer F.Cu) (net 10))
 (segment (start 124.053006 74.356216) (end 123.35622 75.053002) (width 0.2) (layer F.Cu) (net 10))
 (segment (start 124.053006 72.053006) (end 124.053006 74.356216) (width 0.2) (layer F.Cu) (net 10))
 (segment (start 123 71) (end 124.053006 72.053006) (width 0.2) (layer F.Cu) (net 10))
 (segment (start 119.5 71) (end 123 71) (width 0.2) (layer F.Cu) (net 10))
 (segment (start 118.5 72) (end 119.5 71) (width 0.2) (layer F.Cu) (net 10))
 (segment (start 118.5 82.5) (end 118.5 72) (width 0.2) (layer F.Cu) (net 10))
 (segment (start 116.446998 84.553002) (end 118.5 82.5) (width 0.2) (layer F.Cu) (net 10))
 (segment (start 113.053002 84.553002) (end 116.446998 84.553002) (width 0.2) (layer F.Cu) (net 10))
 (segment (start 108 79.5) (end 113.053002 84.553002) (width 0.2) (layer F.Cu) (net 10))
 (segment (start 111 85.5) (end 108 82.5) (width 0.2) (layer F.Cu) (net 9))
 (segment (start 117 85.5) (end 111 85.5) (width 0.2) (layer F.Cu) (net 9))
 (segment (start 119 83.5) (end 117 85.5) (width 0.2) (layer F.Cu) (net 9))
 (segment (start 119 75.7875) (end 119 83.5) (width 0.2) (layer F.Cu) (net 9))
 (segment (start 119 74.7875) (end 119 75.7875) (width 0.2) (layer F.Cu) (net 9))
 (segment (start 120 73.7875) (end 119 74.7875) (width 0.2) (layer F.Cu) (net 9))
 (segment (start 120 82.5) (end 120 81.7875) (width 0.2) (layer F.Cu) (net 12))
 (segment (start 120 82.2875) (end 120 82.5) (width 0.2) (layer F.Cu) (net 12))
 (segment (start 109.5 87) (end 108 85.5) (width 0.2) (layer F.Cu) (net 12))
 (segment (start 116.7875 87) (end 109.5 87) (width 0.2) (layer F.Cu) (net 12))
 (segment (start 120 83.7875) (end 116.7875 87) (width 0.2) (layer F.Cu) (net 12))
 (segment (start 120 81.7875) (end 120 83.7875) (width 0.2) (layer F.Cu) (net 12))
 (segment (start 111.2125 88.5) (end 108 88.5) (width 0.2) (layer F.Cu) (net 15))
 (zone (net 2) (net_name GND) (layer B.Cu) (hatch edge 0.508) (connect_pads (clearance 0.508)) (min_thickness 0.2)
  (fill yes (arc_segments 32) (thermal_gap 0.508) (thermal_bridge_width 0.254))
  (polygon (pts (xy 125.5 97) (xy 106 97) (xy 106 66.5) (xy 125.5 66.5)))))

